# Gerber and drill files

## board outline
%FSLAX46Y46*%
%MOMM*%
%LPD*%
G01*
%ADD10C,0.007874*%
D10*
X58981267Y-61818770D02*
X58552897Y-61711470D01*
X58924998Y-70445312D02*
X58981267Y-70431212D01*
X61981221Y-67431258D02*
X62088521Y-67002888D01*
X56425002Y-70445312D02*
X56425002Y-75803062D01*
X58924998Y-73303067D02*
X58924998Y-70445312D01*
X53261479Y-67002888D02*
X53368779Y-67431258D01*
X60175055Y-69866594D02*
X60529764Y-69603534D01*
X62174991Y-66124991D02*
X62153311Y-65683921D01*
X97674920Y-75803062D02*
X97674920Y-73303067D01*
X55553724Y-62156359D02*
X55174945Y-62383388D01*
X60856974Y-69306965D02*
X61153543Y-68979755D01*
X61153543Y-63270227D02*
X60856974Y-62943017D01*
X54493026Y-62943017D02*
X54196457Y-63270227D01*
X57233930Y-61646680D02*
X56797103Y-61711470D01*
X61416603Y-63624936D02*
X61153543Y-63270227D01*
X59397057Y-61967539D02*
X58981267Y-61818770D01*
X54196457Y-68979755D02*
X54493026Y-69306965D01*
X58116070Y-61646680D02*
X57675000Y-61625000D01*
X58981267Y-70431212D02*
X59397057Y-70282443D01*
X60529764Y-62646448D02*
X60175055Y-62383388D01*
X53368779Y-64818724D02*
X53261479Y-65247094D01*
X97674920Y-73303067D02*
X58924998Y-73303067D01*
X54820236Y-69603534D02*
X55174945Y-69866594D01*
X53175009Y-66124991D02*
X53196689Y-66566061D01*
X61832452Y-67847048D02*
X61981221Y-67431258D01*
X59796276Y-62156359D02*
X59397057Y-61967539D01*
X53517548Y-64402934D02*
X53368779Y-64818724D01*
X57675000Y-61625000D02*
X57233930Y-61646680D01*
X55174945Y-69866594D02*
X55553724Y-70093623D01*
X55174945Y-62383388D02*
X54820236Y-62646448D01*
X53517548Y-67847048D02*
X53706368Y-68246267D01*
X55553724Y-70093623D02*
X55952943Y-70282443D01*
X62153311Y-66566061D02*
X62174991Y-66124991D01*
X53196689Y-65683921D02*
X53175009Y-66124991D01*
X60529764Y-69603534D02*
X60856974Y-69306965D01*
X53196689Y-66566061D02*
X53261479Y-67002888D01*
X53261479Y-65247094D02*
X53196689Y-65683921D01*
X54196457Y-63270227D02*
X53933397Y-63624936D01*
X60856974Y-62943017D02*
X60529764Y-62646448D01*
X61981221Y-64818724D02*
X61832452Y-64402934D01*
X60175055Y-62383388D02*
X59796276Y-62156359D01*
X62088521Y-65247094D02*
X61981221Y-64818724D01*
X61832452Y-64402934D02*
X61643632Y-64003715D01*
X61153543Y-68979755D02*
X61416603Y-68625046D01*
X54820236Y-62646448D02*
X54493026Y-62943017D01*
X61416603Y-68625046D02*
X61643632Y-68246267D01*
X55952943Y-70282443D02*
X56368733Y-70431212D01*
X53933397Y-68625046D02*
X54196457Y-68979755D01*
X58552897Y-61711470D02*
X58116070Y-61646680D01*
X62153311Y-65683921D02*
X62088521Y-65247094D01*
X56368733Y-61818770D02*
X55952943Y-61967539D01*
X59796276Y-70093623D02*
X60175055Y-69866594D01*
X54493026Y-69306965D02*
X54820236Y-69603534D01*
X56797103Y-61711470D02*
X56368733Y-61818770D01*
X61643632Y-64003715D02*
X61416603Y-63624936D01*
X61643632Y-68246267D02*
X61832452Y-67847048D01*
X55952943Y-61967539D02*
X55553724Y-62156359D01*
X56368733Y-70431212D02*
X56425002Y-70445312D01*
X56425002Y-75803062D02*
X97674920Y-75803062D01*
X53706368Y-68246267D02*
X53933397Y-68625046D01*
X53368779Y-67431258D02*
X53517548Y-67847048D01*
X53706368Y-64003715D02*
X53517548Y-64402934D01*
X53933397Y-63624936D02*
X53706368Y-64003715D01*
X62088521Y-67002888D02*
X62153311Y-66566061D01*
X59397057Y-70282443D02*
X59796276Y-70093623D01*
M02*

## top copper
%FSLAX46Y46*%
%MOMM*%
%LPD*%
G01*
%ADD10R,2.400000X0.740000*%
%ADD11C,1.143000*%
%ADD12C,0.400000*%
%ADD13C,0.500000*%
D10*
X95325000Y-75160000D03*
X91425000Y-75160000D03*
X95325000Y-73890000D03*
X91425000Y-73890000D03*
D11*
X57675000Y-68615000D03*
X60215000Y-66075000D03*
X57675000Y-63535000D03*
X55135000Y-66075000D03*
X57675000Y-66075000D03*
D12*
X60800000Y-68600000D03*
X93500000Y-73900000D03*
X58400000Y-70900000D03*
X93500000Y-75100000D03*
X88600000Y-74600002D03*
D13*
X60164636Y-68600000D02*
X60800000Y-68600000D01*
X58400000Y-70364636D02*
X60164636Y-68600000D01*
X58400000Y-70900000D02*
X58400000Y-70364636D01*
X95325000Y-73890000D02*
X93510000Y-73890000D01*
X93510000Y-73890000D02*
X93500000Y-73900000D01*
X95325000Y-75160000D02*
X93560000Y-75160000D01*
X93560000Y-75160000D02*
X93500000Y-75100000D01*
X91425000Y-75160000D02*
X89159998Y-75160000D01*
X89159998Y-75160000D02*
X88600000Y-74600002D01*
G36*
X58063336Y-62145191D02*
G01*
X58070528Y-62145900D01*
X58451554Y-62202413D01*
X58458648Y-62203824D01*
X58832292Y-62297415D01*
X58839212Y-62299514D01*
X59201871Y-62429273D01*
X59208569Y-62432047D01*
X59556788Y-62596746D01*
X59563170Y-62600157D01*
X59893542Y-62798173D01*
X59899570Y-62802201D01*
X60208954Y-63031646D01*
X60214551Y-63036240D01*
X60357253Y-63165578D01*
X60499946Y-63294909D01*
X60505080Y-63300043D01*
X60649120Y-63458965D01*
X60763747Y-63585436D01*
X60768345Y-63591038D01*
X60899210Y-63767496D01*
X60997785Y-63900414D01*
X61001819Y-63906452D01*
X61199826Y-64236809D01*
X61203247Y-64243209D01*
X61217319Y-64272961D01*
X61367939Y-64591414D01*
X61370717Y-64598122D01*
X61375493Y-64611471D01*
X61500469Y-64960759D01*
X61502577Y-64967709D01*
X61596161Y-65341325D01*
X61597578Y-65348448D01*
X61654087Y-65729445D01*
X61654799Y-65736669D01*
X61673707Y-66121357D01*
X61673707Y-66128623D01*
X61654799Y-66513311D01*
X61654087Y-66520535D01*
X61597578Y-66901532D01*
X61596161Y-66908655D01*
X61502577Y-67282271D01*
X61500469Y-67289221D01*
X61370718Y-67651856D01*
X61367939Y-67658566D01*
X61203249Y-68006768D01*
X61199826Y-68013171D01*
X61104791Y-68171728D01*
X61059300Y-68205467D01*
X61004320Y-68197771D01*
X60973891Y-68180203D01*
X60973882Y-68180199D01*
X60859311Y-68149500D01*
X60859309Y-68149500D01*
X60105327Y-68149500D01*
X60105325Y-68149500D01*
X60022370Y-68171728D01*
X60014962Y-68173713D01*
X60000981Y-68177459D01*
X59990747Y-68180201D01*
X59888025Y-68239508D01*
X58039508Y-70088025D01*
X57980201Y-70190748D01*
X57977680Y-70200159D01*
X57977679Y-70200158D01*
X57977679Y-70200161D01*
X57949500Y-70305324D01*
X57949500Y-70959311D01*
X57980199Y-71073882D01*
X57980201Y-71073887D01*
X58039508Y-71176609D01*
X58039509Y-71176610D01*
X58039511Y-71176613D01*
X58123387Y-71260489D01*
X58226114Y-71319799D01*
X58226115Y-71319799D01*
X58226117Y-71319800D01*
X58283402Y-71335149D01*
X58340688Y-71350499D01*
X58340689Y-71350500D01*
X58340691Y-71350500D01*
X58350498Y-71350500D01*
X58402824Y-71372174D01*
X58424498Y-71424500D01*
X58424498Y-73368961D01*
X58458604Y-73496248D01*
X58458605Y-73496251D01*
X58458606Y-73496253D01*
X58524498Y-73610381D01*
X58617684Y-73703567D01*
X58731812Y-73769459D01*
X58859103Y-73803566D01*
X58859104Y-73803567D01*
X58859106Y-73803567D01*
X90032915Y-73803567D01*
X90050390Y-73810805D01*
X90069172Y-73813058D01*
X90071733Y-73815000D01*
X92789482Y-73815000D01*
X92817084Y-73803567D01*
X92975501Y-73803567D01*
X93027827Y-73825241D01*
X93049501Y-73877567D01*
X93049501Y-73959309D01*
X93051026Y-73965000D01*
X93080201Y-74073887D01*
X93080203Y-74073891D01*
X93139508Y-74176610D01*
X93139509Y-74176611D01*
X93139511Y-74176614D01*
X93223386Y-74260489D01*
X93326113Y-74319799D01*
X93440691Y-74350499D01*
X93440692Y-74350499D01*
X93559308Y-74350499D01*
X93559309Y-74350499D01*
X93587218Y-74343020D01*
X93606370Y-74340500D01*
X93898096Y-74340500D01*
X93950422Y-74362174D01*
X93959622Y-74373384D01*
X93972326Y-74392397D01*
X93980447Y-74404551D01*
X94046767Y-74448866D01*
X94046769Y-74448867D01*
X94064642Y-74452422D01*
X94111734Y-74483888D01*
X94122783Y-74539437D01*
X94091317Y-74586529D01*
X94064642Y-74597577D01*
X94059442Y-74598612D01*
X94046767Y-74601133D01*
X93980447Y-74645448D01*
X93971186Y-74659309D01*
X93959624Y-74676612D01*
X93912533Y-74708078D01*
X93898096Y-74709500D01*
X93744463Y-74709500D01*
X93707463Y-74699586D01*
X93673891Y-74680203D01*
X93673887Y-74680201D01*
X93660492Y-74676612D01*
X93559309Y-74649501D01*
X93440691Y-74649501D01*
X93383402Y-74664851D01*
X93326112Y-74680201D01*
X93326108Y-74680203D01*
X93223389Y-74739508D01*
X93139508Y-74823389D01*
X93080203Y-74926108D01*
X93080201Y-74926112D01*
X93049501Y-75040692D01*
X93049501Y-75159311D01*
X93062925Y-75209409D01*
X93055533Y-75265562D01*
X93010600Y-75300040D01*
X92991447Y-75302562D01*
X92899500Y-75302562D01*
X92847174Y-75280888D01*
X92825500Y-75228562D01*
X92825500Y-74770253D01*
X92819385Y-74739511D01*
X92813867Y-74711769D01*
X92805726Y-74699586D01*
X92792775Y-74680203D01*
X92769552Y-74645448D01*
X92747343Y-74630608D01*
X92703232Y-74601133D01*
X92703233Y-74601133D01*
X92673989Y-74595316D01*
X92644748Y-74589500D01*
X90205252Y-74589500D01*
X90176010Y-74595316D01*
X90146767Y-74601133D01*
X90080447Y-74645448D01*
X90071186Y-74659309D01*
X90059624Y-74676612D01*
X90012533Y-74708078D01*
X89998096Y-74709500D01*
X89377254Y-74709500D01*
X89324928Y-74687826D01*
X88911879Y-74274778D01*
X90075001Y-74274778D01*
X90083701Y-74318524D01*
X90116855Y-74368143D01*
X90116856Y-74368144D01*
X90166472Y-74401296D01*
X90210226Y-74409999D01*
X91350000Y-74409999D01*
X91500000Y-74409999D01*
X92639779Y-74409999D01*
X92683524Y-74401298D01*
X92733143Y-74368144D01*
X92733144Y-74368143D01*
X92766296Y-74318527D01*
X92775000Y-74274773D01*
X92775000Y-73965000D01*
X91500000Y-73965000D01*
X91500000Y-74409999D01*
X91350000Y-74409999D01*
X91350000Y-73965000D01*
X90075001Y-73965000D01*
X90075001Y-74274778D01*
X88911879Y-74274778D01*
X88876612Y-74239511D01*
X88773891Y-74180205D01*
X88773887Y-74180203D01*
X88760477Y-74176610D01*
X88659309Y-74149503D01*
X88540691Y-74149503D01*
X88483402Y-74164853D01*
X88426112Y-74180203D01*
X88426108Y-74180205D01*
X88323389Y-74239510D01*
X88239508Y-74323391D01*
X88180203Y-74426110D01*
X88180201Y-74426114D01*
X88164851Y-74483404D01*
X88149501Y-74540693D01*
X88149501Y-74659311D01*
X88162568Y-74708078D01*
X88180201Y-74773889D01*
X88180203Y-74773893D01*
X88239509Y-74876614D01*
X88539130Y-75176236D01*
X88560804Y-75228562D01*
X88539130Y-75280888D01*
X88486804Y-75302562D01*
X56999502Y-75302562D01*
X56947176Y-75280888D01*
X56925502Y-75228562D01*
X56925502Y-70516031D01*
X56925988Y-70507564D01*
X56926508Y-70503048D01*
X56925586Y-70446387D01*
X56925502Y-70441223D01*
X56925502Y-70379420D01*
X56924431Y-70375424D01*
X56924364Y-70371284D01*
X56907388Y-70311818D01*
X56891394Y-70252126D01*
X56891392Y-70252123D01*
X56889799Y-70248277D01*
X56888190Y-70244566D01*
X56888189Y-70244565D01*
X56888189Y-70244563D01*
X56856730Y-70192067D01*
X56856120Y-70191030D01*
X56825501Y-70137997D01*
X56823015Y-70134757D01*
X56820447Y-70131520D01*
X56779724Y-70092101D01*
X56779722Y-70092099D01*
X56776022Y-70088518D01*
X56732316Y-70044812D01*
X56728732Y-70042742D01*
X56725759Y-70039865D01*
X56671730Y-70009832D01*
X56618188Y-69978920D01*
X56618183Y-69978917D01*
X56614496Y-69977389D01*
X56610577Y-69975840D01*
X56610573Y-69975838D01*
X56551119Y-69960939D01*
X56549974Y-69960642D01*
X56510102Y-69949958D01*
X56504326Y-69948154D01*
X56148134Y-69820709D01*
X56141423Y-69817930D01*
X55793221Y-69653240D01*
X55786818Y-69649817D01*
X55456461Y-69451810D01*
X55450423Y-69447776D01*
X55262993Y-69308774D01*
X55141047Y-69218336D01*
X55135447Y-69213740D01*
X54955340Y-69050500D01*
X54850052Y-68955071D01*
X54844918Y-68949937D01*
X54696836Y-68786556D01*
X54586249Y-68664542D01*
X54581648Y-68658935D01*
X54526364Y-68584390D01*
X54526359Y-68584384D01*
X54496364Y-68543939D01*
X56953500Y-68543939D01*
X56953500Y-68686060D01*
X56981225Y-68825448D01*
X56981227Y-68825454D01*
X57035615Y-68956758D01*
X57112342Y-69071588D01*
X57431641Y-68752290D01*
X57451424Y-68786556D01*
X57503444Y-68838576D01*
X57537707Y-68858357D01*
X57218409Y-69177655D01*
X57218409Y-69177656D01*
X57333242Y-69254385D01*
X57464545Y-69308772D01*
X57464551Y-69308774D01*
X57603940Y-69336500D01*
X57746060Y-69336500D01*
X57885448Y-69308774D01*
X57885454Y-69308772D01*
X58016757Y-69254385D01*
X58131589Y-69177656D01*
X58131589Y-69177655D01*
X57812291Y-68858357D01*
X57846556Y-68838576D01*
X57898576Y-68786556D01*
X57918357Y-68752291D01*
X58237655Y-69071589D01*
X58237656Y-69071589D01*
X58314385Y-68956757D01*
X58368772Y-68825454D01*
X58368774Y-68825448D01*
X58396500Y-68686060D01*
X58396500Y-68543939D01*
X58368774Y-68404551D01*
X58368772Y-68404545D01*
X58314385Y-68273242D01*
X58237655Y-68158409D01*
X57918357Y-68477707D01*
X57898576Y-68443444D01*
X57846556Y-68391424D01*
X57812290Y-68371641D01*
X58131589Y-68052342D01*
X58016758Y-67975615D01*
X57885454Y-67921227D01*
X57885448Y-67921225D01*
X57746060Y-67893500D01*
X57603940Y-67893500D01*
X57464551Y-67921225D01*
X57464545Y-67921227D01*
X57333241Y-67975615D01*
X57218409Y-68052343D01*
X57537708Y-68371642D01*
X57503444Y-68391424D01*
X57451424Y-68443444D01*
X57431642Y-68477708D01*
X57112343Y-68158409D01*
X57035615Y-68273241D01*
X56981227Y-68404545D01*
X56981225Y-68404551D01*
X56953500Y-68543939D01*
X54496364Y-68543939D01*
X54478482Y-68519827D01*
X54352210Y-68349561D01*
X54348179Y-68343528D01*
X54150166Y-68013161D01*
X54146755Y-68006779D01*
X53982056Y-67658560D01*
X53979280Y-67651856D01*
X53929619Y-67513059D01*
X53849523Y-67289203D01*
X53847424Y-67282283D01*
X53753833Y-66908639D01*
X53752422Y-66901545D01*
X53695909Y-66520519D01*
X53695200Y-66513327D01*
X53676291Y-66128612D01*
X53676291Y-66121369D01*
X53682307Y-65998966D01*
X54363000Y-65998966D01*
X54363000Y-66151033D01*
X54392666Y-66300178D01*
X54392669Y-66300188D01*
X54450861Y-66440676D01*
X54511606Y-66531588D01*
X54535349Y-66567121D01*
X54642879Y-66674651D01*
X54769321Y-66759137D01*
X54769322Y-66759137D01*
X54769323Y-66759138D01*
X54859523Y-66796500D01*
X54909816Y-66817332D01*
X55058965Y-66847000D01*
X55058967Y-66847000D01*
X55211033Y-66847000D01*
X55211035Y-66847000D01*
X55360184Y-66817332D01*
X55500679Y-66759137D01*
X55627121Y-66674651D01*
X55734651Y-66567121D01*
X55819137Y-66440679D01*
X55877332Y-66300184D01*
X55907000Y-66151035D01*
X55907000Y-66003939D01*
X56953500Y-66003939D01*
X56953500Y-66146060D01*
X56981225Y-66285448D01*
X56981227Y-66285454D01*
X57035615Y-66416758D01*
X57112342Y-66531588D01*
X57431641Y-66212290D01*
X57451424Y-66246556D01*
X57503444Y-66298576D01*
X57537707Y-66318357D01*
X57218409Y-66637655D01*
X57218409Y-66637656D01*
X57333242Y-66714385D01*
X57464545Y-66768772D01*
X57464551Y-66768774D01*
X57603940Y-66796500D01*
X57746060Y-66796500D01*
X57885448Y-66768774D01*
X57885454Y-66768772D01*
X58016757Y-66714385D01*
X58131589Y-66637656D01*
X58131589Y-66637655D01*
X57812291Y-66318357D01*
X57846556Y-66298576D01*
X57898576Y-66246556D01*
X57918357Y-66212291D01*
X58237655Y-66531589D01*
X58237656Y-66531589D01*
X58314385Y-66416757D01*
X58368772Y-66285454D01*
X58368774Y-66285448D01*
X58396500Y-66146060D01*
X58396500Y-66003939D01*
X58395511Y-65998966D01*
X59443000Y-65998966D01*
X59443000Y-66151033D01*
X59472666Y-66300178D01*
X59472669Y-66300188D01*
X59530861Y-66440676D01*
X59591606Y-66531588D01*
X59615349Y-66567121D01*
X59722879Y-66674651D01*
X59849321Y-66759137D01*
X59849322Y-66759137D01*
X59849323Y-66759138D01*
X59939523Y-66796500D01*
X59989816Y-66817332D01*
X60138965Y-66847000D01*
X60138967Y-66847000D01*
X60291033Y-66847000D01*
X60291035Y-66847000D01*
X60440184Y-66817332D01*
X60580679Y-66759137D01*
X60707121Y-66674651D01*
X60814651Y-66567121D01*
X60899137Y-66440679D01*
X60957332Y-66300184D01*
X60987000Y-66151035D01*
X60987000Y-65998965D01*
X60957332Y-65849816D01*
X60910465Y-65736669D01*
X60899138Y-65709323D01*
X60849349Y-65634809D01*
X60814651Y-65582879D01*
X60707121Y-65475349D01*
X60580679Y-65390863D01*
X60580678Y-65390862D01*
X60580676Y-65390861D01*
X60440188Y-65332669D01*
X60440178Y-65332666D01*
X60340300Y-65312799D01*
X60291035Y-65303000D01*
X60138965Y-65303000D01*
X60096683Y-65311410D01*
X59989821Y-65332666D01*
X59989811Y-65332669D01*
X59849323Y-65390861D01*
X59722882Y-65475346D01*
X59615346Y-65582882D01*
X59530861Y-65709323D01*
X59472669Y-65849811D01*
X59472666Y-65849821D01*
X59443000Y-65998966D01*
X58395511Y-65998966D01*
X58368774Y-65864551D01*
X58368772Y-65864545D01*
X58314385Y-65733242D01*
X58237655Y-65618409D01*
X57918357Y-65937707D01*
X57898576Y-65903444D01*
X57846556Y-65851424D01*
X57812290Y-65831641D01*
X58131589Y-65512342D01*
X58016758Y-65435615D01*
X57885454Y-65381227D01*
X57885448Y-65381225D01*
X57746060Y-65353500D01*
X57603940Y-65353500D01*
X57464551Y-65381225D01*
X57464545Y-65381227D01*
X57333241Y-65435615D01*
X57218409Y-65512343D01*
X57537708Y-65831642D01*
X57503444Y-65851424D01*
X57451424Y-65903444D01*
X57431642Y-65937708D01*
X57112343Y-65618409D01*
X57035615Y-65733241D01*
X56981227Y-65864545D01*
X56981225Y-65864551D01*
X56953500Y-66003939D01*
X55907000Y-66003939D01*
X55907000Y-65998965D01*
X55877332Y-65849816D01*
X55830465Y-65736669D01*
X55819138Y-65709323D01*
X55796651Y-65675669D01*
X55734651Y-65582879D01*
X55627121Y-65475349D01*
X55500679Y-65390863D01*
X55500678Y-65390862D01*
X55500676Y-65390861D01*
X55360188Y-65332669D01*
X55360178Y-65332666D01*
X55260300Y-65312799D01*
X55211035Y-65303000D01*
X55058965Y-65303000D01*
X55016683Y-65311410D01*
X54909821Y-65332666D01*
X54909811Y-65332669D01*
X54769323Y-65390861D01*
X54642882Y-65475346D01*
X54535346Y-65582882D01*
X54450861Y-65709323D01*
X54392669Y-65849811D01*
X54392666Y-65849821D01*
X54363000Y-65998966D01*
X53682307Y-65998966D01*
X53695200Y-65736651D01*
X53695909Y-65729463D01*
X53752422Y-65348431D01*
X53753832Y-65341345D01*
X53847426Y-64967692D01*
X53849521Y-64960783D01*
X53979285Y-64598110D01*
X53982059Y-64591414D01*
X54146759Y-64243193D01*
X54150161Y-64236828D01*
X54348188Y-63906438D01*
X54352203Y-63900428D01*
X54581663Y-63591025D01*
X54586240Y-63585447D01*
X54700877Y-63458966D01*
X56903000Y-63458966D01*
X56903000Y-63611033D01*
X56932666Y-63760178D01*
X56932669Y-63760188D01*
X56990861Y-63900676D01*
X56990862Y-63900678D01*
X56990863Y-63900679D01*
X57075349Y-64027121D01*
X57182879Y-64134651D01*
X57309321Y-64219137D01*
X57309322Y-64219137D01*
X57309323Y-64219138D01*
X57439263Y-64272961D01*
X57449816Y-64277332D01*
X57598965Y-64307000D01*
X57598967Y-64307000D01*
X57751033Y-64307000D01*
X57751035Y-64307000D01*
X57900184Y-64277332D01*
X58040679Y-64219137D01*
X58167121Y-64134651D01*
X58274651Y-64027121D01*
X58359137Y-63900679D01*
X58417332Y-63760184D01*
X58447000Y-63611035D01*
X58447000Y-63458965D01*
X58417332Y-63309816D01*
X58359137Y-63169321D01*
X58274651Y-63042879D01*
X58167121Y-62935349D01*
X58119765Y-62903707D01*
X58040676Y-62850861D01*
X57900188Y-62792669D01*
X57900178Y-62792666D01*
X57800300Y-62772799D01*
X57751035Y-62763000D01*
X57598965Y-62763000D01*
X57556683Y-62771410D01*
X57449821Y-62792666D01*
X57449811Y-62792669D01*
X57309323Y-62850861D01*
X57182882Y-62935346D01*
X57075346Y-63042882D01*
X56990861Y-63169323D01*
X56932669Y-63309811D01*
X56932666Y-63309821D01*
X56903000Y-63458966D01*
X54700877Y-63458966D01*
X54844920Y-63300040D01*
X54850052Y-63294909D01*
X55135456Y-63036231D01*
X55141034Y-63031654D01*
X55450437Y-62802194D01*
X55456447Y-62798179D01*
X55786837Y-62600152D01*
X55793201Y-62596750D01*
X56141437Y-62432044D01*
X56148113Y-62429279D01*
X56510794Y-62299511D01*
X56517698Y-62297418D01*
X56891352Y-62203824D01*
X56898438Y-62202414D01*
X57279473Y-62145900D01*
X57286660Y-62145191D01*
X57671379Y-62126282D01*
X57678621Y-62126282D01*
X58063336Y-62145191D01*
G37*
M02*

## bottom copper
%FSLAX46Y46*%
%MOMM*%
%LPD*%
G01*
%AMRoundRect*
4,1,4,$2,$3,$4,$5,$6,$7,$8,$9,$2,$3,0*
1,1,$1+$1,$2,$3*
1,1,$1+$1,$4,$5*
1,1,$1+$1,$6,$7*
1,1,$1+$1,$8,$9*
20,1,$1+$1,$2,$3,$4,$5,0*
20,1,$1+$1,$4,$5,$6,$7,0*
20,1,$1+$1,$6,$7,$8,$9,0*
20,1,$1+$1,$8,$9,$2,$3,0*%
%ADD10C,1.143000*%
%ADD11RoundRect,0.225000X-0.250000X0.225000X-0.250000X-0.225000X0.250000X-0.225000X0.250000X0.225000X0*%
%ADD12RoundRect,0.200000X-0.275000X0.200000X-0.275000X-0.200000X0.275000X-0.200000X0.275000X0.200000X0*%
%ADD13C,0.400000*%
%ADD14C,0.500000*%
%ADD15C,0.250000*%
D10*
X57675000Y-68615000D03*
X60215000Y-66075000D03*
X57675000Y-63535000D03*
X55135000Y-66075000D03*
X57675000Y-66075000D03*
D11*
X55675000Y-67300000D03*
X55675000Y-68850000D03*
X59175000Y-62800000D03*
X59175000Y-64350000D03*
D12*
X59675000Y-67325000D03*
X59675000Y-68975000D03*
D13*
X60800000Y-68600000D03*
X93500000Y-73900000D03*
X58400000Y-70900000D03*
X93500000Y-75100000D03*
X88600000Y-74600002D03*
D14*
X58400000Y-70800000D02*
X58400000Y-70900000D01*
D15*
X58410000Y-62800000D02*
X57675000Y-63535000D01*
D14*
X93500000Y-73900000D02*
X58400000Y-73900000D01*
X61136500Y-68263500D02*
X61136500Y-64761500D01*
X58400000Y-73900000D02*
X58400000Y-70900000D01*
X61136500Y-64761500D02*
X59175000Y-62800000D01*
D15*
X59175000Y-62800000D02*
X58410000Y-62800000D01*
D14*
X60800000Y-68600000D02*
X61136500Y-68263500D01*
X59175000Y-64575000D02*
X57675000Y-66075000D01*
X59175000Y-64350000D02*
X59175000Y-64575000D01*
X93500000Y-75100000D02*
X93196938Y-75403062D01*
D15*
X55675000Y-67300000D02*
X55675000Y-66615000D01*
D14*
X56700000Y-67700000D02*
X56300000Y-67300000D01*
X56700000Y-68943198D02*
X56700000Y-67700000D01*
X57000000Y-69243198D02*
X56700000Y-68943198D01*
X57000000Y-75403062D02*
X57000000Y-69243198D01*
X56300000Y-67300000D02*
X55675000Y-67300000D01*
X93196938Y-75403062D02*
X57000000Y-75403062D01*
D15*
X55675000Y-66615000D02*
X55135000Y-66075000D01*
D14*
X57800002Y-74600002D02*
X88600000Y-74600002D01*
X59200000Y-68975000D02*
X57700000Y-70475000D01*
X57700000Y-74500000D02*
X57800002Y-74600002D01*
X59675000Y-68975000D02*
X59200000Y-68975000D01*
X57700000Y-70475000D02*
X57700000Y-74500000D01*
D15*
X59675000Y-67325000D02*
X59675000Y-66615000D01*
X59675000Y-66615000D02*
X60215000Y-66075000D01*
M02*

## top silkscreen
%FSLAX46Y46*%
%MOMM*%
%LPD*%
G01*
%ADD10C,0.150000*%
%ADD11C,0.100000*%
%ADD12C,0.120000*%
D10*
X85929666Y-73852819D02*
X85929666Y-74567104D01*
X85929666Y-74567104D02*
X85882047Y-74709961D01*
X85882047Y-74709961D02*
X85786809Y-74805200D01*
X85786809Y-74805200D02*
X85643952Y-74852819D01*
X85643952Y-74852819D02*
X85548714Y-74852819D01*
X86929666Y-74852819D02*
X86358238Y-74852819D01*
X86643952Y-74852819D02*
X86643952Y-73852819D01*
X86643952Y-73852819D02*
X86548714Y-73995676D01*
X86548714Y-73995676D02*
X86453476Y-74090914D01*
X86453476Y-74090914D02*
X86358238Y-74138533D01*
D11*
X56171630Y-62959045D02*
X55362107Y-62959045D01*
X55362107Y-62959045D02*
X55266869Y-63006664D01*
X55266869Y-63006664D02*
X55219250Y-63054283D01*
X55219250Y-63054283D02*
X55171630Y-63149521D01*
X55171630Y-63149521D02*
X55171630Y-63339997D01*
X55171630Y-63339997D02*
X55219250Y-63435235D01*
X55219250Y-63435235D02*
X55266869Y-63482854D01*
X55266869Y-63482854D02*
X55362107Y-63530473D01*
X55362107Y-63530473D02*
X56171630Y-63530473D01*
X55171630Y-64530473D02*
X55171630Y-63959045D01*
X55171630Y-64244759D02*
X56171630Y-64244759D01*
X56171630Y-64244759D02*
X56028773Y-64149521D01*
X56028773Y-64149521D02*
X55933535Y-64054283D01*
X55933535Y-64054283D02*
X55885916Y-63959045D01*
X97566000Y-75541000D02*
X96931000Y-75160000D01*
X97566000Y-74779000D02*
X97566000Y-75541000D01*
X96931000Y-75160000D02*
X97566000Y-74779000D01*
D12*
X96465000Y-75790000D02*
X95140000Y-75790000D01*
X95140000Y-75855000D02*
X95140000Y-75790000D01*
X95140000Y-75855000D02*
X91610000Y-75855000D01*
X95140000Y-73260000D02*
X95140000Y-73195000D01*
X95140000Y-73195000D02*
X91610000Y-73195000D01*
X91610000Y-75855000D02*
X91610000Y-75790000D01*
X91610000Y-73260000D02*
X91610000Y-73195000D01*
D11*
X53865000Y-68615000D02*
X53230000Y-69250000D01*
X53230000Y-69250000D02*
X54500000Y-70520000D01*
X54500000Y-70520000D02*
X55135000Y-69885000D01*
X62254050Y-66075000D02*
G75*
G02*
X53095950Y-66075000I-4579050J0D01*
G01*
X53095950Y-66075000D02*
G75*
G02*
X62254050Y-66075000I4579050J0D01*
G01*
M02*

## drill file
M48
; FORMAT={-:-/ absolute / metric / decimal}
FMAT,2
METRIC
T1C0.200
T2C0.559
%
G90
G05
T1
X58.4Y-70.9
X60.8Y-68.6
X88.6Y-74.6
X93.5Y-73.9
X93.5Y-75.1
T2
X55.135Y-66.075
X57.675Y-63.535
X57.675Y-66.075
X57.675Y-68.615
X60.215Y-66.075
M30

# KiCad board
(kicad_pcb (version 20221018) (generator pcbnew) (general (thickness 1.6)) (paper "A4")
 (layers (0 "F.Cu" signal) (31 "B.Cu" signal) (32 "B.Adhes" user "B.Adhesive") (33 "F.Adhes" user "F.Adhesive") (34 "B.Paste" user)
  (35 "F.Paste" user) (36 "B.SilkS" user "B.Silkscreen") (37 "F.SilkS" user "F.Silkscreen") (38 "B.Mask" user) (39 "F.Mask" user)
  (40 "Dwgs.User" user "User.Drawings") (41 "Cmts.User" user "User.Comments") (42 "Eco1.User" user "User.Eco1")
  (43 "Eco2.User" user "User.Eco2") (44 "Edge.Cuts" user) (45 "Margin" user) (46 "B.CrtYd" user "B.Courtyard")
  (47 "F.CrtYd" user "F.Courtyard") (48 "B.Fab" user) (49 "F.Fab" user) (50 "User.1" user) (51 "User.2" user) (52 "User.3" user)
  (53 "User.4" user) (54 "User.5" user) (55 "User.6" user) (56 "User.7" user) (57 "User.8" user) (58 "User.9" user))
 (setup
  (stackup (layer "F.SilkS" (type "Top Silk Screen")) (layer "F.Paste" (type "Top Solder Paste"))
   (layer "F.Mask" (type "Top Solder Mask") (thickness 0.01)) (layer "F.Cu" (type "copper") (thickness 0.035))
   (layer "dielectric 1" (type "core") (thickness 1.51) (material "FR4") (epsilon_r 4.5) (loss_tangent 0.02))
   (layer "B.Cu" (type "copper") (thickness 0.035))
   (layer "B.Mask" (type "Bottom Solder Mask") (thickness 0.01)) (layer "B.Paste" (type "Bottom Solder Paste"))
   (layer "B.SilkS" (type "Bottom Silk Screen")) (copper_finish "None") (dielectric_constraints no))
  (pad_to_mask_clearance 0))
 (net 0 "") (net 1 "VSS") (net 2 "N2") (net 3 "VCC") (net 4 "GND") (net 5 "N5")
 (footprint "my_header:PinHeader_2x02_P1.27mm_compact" (layer "F.Cu") (at 93.375 74.525 180)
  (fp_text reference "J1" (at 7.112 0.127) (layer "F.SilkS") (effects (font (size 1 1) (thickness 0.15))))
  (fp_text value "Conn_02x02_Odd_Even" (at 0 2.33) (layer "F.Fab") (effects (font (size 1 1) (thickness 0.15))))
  (fp_line (start -4.191 -1.016) (end -3.556 -0.635) (stroke (width 0.1) (type default)) (layer "F.SilkS"))
  (fp_line (start -4.191 -0.254) (end -4.191 -1.016) (stroke (width 0.1) (type default)) (layer "F.SilkS"))
  (fp_line (start -3.556 -0.635) (end -4.191 -0.254) (stroke (width 0.1) (type default)) (layer "F.SilkS"))
  (fp_line (start -3.09 -1.265) (end -1.765 -1.265) (stroke (width 0.12) (type solid)) (layer "F.SilkS"))
  (fp_line (start -1.765 -1.33) (end -1.765 -1.265) (stroke (width 0.12) (type solid)) (layer "F.SilkS"))
  (fp_line (start -1.765 -1.33) (end 1.765 -1.33) (stroke (width 0.12) (type solid)) (layer "F.SilkS"))
  (fp_line (start -1.765 1.265) (end -1.765 1.33) (stroke (width 0.12) (type solid)) (layer "F.SilkS"))
  (fp_line (start -1.765 1.33) (end 1.765 1.33) (stroke (width 0.12) (type solid)) (layer "F.SilkS"))
  (fp_line (start 1.765 -1.33) (end 1.765 -1.265) (stroke (width 0.12) (type solid)) (layer "F.SilkS"))
  (fp_line (start 1.765 1.265) (end 1.765 1.33) (stroke (width 0.12) (type solid)) (layer "F.SilkS"))
  (pad "1" smd rect (at -1.95 -0.635 180) (size 2.4 0.74) (layers "F.Cu" "F.Paste" "F.Mask") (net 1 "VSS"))
  (pad "2" smd rect (at 1.95 -0.635 180) (size 2.4 0.74) (layers "F.Cu" "F.Paste" "F.Mask") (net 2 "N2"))
  (pad "3" smd rect (at -1.95 0.635 180) (size 2.4 0.74) (layers "F.Cu" "F.Paste" "F.Mask") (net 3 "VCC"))
  (pad "4" smd rect (at 1.95 0.635 180) (size 2.4 0.74) (layers "F.Cu" "F.Paste" "F.Mask") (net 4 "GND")))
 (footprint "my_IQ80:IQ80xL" (layer "F.Cu") (at 57.675 63.535 -90)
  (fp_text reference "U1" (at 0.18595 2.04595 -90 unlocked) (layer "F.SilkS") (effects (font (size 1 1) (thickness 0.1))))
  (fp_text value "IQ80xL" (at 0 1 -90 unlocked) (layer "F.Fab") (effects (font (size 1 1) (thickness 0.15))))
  (fp_line (start 5.08 3.81) (end 5.715 4.445) (stroke (width 0.1) (type default)) (layer "F.SilkS"))
  (fp_line (start 5.715 4.445) (end 6.985 3.175) (stroke (width 0.1) (type default)) (layer "F.SilkS"))
  (fp_line (start 6.985 3.175) (end 6.35 2.54) (stroke (width 0.1) (type default)) (layer "F.SilkS"))
  (fp_circle (center 2.54 0) (end 6.35 2.54) (stroke (width 0.1) (type default)) (fill none) (layer "F.SilkS"))
  (pad "1" thru_hole circle (at 5.08 0 270) (size 1.143 1.143) (drill 0.5588) (layers "*.Cu" "*.Mask") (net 4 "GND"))
  (pad "2" thru_hole circle (at 2.54 -2.54 270) (size 1.143 1.143) (drill 0.5588) (layers "*.Cu" "*.Mask") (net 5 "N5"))
  (pad "3" thru_hole circle (at 0 0 270) (size 1.143 1.143) (drill 0.5588) (layers "*.Cu" "*.Mask") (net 3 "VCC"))
  (pad "4" thru_hole circle (at 2.54 2.54 270) (size 1.143 1.143) (drill 0.5588) (layers "*.Cu" "*.Mask") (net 1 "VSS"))
  (pad "5" thru_hole circle (at 2.54 0 270) (size 1.143 1.143) (drill 0.5588) (layers "*.Cu" "*.Mask") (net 4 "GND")))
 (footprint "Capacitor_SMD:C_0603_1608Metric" (layer "B.Cu") (at 55.675 68.075 -90)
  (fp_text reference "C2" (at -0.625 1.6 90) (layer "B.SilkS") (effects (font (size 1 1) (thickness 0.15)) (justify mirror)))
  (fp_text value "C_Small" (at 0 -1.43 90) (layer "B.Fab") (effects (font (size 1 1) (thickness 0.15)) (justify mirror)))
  (pad "1" smd roundrect (at -0.775 0 270) (size 0.9 0.95) (layers "B.Cu" "B.Paste" "B.Mask") (roundrect_rratio 0.25) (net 1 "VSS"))
  (pad "2" smd roundrect (at 0.775 0 270) (size 0.9 0.95) (layers "B.Cu" "B.Paste" "B.Mask") (roundrect_rratio 0.25) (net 4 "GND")))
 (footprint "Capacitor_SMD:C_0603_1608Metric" (layer "B.Cu") (at 59.175 63.575 -90)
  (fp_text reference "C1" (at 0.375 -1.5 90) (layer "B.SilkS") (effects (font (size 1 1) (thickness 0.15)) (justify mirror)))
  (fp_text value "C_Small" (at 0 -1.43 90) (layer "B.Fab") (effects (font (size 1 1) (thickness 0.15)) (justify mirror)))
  (pad "1" smd roundrect (at -0.775 0 270) (size 0.9 0.95) (layers "B.Cu" "B.Paste" "B.Mask") (roundrect_rratio 0.25) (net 3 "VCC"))
  (pad "2" smd roundrect (at 0.775 0 270) (size 0.9 0.95) (layers "B.Cu" "B.Paste" "B.Mask") (roundrect_rratio 0.25) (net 4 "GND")))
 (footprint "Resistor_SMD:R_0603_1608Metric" (layer "B.Cu") (at 59.675 68.15 -90)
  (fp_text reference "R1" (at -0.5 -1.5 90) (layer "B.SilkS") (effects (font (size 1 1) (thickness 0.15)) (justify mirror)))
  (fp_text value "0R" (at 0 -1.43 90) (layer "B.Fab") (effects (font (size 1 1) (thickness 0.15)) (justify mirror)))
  (pad "1" smd roundrect (at -0.825 0 270) (size 0.8 0.95) (layers "B.Cu" "B.Paste" "B.Mask") (roundrect_rratio 0.25) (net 5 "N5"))
  (pad "2" smd roundrect (at 0.825 0 270) (size 0.8 0.95) (layers "B.Cu" "B.Paste" "B.Mask") (roundrect_rratio 0.25) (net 2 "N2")))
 (gr_line (start 58.981267 61.81877) (end 58.552897 61.71147) (stroke (width 0.007874) (type solid)) (layer "Edge.Cuts"))
 (gr_line (start 58.924998 70.445312) (end 58.981267 70.431212) (stroke (width 0.007874) (type solid)) (layer "Edge.Cuts"))
 (gr_line (start 61.981221 67.431258) (end 62.088521 67.002888) (stroke (width 0.007874) (type solid)) (layer "Edge.Cuts"))
 (gr_line (start 56.425002 70.445312) (end 56.425002 75.803062) (stroke (width 0.007874) (type solid)) (layer "Edge.Cuts"))
 (gr_line (start 58.924998 73.303067) (end 58.924998 70.445312) (stroke (width 0.007874) (type solid)) (layer "Edge.Cuts"))
 (gr_line (start 53.261479 67.002888) (end 53.368779 67.431258) (stroke (width 0.007874) (type solid)) (layer "Edge.Cuts"))
 (gr_line (start 60.175055 69.866594) (end 60.529764 69.603534) (stroke (width 0.007874) (type solid)) (layer "Edge.Cuts"))
 (gr_line (start 62.174991 66.124991) (end 62.153311 65.683921) (stroke (width 0.007874) (type solid)) (layer "Edge.Cuts"))
 (gr_line (start 97.67492 75.803062) (end 97.67492 73.303067) (stroke (width 0.007874) (type solid)) (layer "Edge.Cuts"))
 (gr_line (start 55.553724 62.156359) (end 55.174945 62.383388) (stroke (width 0.007874) (type solid)) (layer "Edge.Cuts"))
 (gr_line (start 60.856974 69.306965) (end 61.153543 68.979755) (stroke (width 0.007874) (type solid)) (layer "Edge.Cuts"))
 (gr_line (start 61.153543 63.270227) (end 60.856974 62.943017) (stroke (width 0.007874) (type solid)) (layer "Edge.Cuts"))
 (gr_line (start 54.493026 62.943017) (end 54.196457 63.270227) (stroke (width 0.007874) (type solid)) (layer "Edge.Cuts"))
 (gr_line (start 57.23393 61.64668) (end 56.797103 61.71147) (stroke (width 0.007874) (type solid)) (layer "Edge.Cuts"))
 (gr_line (start 61.416603 63.624936) (end 61.153543 63.270227) (stroke (width 0.007874) (type solid)) (layer "Edge.Cuts"))
 (gr_line (start 59.397057 61.967539) (end 58.981267 61.81877) (stroke (width 0.007874) (type solid)) (layer "Edge.Cuts"))
 (gr_line (start 54.196457 68.979755) (end 54.493026 69.306965) (stroke (width 0.007874) (type solid)) (layer "Edge.Cuts"))
 (gr_line (start 58.11607 61.64668) (end 57.675 61.625) (stroke (width 0.007874) (type solid)) (layer "Edge.Cuts"))
 (gr_line (start 58.981267 70.431212) (end 59.397057 70.282443) (stroke (width 0.007874) (type solid)) (layer "Edge.Cuts"))
 (gr_line (start 60.529764 62.646448) (end 60.175055 62.383388) (stroke (width 0.007874) (type solid)) (layer "Edge.Cuts"))
 (gr_line (start 53.368779 64.818724) (end 53.261479 65.247094) (stroke (width 0.007874) (type solid)) (layer "Edge.Cuts"))
 (gr_line (start 97.67492 73.303067) (end 58.924998 73.303067) (stroke (width 0.007874) (type solid)) (layer "Edge.Cuts"))
 (gr_line (start 54.820236 69.603534) (end 55.174945 69.866594) (stroke (width 0.007874) (type solid)) (layer "Edge.Cuts"))
 (gr_line (start 53.175009 66.124991) (end 53.196689 66.566061) (stroke (width 0.007874) (type solid)) (layer "Edge.Cuts"))
 (gr_line (start 61.832452 67.847048) (end 61.981221 67.431258) (stroke (width 0.007874) (type solid)) (layer "Edge.Cuts"))
 (gr_line (start 59.796276 62.156359) (end 59.397057 61.967539) (stroke (width 0.007874) (type solid)) (layer "Edge.Cuts"))
 (gr_line (start 53.517548 64.402934) (end 53.368779 64.818724) (stroke (width 0.007874) (type solid)) (layer "Edge.Cuts"))
 (gr_line (start 57.675 61.625) (end 57.23393 61.64668) (stroke (width 0.007874) (type solid)) (layer "Edge.Cuts"))
 (gr_line (start 55.174945 69.866594) (end 55.553724 70.093623) (stroke (width 0.007874) (type solid)) (layer "Edge.Cuts"))
 (gr_line (start 55.174945 62.383388) (end 54.820236 62.646448) (stroke (width 0.007874) (type solid)) (layer "Edge.Cuts"))
 (gr_line (start 53.517548 67.847048) (end 53.706368 68.246267) (stroke (width 0.007874) (type solid)) (layer "Edge.Cuts"))
 (gr_line (start 55.553724 70.093623) (end 55.952943 70.282443) (stroke (width 0.007874) (type solid)) (layer "Edge.Cuts"))
 (gr_line (start 62.153311 66.566061) (end 62.174991 66.124991) (stroke (width 0.007874) (type solid)) (layer "Edge.Cuts"))
 (gr_line (start 53.196689 65.683921) (end 53.175009 66.124991) (stroke (width 0.007874) (type solid)) (layer "Edge.Cuts"))
 (gr_line (start 60.529764 69.603534) (end 60.856974 69.306965) (stroke (width 0.007874) (type solid)) (layer "Edge.Cuts"))
 (gr_line (start 53.196689 66.566061) (end 53.261479 67.002888) (stroke (width 0.007874) (type solid)) (layer "Edge.Cuts"))
 (gr_line (start 53.261479 65.247094) (end 53.196689 65.683921) (stroke (width 0.007874) (type solid)) (layer "Edge.Cuts"))
 (gr_line (start 54.196457 63.270227) (end 53.933397 63.624936) (stroke (width 0.007874) (type solid)) (layer "Edge.Cuts"))
 (gr_line (start 60.856974 62.943017) (end 60.529764 62.646448) (stroke (width 0.007874) (type solid)) (layer "Edge.Cuts"))
 (gr_line (start 61.981221 64.818724) (end 61.832452 64.402934) (stroke (width 0.007874) (type solid)) (layer "Edge.Cuts"))
 (gr_line (start 60.175055 62.383388) (end 59.796276 62.156359) (stroke (width 0.007874) (type solid)) (layer "Edge.Cuts"))
 (gr_line (start 62.088521 65.247094) (end 61.981221 64.818724) (stroke (width 0.007874) (type solid)) (layer "Edge.Cuts"))
 (gr_line (start 61.832452 64.402934) (end 61.643632 64.003715) (stroke (width 0.007874) (type solid)) (layer "Edge.Cuts"))
 (gr_line (start 61.153543 68.979755) (end 61.416603 68.625046) (stroke (width 0.007874) (type solid)) (layer "Edge.Cuts"))
 (gr_line (start 54.820236 62.646448) (end 54.493026 62.943017) (stroke (width 0.007874) (type solid)) (layer "Edge.Cuts"))
 (gr_line (start 61.416603 68.625046) (end 61.643632 68.246267) (stroke (width 0.007874) (type solid)) (layer "Edge.Cuts"))
 (gr_line (start 55.952943 70.282443) (end 56.368733 70.431212) (stroke (width 0.007874) (type solid)) (layer "Edge.Cuts"))
 (gr_line (start 53.933397 68.625046) (end 54.196457 68.979755) (stroke (width 0.007874) (type solid)) (layer "Edge.Cuts"))
 (gr_line (start 58.552897 61.71147) (end 58.11607 61.64668) (stroke (width 0.007874) (type solid)) (layer "Edge.Cuts"))
 (gr_line (start 62.153311 65.683921) (end 62.088521 65.247094) (stroke (width 0.007874) (type solid)) (layer "Edge.Cuts"))
 (gr_line (start 56.368733 61.81877) (end 55.952943 61.967539) (stroke (width 0.007874) (type solid)) (layer "Edge.Cuts"))
 (gr_line (start 59.796276 70.093623) (end 60.175055 69.866594) (stroke (width 0.007874) (type solid)) (layer "Edge.Cuts"))
 (gr_line (start 54.493026 69.306965) (end 54.820236 69.603534) (stroke (width 0.007874) (type solid)) (layer "Edge.Cuts"))
 (gr_line (start 56.797103 61.71147) (end 56.368733 61.81877) (stroke (width 0.007874) (type solid)) (layer "Edge.Cuts"))
 (gr_line (start 61.643632 64.003715) (end 61.416603 63.624936) (stroke (width 0.007874) (type solid)) (layer "Edge.Cuts"))
 (gr_line (start 61.643632 68.246267) (end 61.832452 67.847048) (stroke (width 0.007874) (type solid)) (layer "Edge.Cuts"))
 (gr_line (start 55.952943 61.967539) (end 55.553724 62.156359) (stroke (width 0.007874) (type solid)) (layer "Edge.Cuts"))
 (gr_line (start 56.368733 70.431212) (end 56.425002 70.445312) (stroke (width 0.007874) (type solid)) (layer "Edge.Cuts"))
 (gr_line (start 56.425002 75.803062) (end 97.67492 75.803062) (stroke (width 0.007874) (type solid)) (layer "Edge.Cuts"))
 (gr_line (start 53.706368 68.246267) (end 53.933397 68.625046) (stroke (width 0.007874) (type solid)) (layer "Edge.Cuts"))
 (gr_line (start 53.368779 67.431258) (end 53.517548 67.847048) (stroke (width 0.007874) (type solid)) (layer "Edge.Cuts"))
 (gr_line (start 53.706368 64.003715) (end 53.517548 64.402934) (stroke (width 0.007874) (type solid)) (layer "Edge.Cuts"))
 (gr_line (start 53.933397 63.624936) (end 53.706368 64.003715) (stroke (width 0.007874) (type solid)) (layer "Edge.Cuts"))
 (gr_line (start 62.088521 67.002888) (end 62.153311 66.566061) (stroke (width 0.007874) (type solid)) (layer "Edge.Cuts"))
 (gr_line (start 59.397057 70.282443) (end 59.796276 70.093623) (stroke (width 0.007874) (type solid)) (layer "Edge.Cuts"))
 (segment (start 60.164636 68.6) (end 60.8 68.6) (width 0.5) (layer "F.Cu") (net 3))
 (segment (start 58.4 70.364636) (end 60.164636 68.6) (width 0.5) (layer "F.Cu") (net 3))
 (segment (start 58.4 70.9) (end 58.4 70.364636) (width 0.5) (layer "F.Cu") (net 3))
 (segment (start 95.325 73.89) (end 93.51 73.89) (width 0.5) (layer "F.Cu") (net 3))
 (segment (start 93.51 73.89) (end 93.5 73.9) (width 0.5) (layer "F.Cu") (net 3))
 (via (at 60.8 68.6) (size 0.4) (drill 0.2) (layers "F.Cu" "B.Cu") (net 3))
 (via (at 93.5 73.9) (size 0.4) (drill 0.2) (layers "F.Cu" "B.Cu") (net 3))
 (via (at 58.4 70.9) (size 0.4) (drill 0.2) (layers "F.Cu" "B.Cu") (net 3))
 (segment (start 58.4 70.8) (end 58.4 70.9) (width 0.5) (layer "B.Cu") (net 3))
 (segment (start 58.41 62.8) (end 57.675 63.535) (width 0.25) (layer "B.Cu") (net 3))
 (segment (start 93.5 73.9) (end 58.4 73.9) (width 0.5) (layer "B.Cu") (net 3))
 (segment (start 61.1365 68.2635) (end 61.1365 64.7615) (width 0.5) (layer "B.Cu") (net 3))
 (segment (start 58.4 73.9) (end 58.4 70.9) (width 0.5) (layer "B.Cu") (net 3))
 (segment (start 61.1365 64.7615) (end 59.175 62.8) (width 0.5) (layer "B.Cu") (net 3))
 (segment (start 59.175 62.8) (end 58.41 62.8) (width 0.25) (layer "B.Cu") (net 3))
 (segment (start 60.8 68.6) (end 61.1365 68.2635) (width 0.5) (layer "B.Cu") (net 3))
 (segment (start 59.175 64.575) (end 57.675 66.075) (width 0.5) (layer "B.Cu") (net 4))
 (segment (start 59.175 64.35) (end 59.175 64.575) (width 0.5) (layer "B.Cu") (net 4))
 (segment (start 95.325 75.16) (end 93.56 75.16) (width 0.5) (layer "F.Cu") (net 1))
 (segment (start 93.56 75.16) (end 93.5 75.1) (width 0.5) (layer "F.Cu") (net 1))
 (via (at 93.5 75.1) (size 0.4) (drill 0.2) (layers "F.Cu" "B.Cu") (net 1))
 (segment (start 93.5 75.1) (end 93.196938 75.403062) (width 0.5) (layer "B.Cu") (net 1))
 (segment (start 55.675 67.3) (end 55.675 66.615) (width 0.25) (layer "B.Cu") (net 1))
 (segment (start 56.7 67.7) (end 56.3 67.3) (width 0.5) (layer "B.Cu") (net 1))
 (segment (start 56.7 68.943198) (end 56.7 67.7) (width 0.5) (layer "B.Cu") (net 1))
 (segment (start 57 69.243198) (end 56.7 68.943198) (width 0.5) (layer "B.Cu") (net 1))
 (segment (start 57 75.403062) (end 57 69.243198) (width 0.5) (layer "B.Cu") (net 1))
 (segment (start 56.3 67.3) (end 55.675 67.3) (width 0.5) (layer "B.Cu") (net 1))
 (segment (start 93.196938 75.403062) (end 57 75.403062) (width 0.5) (layer "B.Cu") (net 1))
 (segment (start 55.675 66.615) (end 55.135 66.075) (width 0.25) (layer "B.Cu") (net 1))
 (segment (start 91.425 75.16) (end 89.159998 75.16) (width 0.5) (layer "F.Cu") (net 2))
 (segment (start 89.159998 75.16) (end 88.6 74.600002) (width 0.5) (layer "F.Cu") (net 2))
 (via (at 88.6 74.600002) (size 0.4) (drill 0.2) (layers "F.Cu" "B.Cu") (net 2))
 (segment (start 57.800002 74.600002) (end 88.6 74.600002) (width 0.5) (layer "B.Cu") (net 2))
 (segment (start 59.2 68.975) (end 57.7 70.475) (width 0.5) (layer "B.Cu") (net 2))
 (segment (start 57.7 74.5) (end 57.800002 74.600002) (width 0.5) (layer "B.Cu") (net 2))
 (segment (start 59.675 68.975) (end 59.2 68.975) (width 0.5) (layer "B.Cu") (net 2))
 (segment (start 57.7 70.475) (end 57.7 74.5) (width 0.5) (layer "B.Cu") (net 2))
 (segment (start 59.675 67.325) (end 59.675 66.615) (width 0.25) (layer "B.Cu") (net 5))
 (segment (start 59.675 66.615) (end 60.215 66.075) (width 0.25) (layer "B.Cu") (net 5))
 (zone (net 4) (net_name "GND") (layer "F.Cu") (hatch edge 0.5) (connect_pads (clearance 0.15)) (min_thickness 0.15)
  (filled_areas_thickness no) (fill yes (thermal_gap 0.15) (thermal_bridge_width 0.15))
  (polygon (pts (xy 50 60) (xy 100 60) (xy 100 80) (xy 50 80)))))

